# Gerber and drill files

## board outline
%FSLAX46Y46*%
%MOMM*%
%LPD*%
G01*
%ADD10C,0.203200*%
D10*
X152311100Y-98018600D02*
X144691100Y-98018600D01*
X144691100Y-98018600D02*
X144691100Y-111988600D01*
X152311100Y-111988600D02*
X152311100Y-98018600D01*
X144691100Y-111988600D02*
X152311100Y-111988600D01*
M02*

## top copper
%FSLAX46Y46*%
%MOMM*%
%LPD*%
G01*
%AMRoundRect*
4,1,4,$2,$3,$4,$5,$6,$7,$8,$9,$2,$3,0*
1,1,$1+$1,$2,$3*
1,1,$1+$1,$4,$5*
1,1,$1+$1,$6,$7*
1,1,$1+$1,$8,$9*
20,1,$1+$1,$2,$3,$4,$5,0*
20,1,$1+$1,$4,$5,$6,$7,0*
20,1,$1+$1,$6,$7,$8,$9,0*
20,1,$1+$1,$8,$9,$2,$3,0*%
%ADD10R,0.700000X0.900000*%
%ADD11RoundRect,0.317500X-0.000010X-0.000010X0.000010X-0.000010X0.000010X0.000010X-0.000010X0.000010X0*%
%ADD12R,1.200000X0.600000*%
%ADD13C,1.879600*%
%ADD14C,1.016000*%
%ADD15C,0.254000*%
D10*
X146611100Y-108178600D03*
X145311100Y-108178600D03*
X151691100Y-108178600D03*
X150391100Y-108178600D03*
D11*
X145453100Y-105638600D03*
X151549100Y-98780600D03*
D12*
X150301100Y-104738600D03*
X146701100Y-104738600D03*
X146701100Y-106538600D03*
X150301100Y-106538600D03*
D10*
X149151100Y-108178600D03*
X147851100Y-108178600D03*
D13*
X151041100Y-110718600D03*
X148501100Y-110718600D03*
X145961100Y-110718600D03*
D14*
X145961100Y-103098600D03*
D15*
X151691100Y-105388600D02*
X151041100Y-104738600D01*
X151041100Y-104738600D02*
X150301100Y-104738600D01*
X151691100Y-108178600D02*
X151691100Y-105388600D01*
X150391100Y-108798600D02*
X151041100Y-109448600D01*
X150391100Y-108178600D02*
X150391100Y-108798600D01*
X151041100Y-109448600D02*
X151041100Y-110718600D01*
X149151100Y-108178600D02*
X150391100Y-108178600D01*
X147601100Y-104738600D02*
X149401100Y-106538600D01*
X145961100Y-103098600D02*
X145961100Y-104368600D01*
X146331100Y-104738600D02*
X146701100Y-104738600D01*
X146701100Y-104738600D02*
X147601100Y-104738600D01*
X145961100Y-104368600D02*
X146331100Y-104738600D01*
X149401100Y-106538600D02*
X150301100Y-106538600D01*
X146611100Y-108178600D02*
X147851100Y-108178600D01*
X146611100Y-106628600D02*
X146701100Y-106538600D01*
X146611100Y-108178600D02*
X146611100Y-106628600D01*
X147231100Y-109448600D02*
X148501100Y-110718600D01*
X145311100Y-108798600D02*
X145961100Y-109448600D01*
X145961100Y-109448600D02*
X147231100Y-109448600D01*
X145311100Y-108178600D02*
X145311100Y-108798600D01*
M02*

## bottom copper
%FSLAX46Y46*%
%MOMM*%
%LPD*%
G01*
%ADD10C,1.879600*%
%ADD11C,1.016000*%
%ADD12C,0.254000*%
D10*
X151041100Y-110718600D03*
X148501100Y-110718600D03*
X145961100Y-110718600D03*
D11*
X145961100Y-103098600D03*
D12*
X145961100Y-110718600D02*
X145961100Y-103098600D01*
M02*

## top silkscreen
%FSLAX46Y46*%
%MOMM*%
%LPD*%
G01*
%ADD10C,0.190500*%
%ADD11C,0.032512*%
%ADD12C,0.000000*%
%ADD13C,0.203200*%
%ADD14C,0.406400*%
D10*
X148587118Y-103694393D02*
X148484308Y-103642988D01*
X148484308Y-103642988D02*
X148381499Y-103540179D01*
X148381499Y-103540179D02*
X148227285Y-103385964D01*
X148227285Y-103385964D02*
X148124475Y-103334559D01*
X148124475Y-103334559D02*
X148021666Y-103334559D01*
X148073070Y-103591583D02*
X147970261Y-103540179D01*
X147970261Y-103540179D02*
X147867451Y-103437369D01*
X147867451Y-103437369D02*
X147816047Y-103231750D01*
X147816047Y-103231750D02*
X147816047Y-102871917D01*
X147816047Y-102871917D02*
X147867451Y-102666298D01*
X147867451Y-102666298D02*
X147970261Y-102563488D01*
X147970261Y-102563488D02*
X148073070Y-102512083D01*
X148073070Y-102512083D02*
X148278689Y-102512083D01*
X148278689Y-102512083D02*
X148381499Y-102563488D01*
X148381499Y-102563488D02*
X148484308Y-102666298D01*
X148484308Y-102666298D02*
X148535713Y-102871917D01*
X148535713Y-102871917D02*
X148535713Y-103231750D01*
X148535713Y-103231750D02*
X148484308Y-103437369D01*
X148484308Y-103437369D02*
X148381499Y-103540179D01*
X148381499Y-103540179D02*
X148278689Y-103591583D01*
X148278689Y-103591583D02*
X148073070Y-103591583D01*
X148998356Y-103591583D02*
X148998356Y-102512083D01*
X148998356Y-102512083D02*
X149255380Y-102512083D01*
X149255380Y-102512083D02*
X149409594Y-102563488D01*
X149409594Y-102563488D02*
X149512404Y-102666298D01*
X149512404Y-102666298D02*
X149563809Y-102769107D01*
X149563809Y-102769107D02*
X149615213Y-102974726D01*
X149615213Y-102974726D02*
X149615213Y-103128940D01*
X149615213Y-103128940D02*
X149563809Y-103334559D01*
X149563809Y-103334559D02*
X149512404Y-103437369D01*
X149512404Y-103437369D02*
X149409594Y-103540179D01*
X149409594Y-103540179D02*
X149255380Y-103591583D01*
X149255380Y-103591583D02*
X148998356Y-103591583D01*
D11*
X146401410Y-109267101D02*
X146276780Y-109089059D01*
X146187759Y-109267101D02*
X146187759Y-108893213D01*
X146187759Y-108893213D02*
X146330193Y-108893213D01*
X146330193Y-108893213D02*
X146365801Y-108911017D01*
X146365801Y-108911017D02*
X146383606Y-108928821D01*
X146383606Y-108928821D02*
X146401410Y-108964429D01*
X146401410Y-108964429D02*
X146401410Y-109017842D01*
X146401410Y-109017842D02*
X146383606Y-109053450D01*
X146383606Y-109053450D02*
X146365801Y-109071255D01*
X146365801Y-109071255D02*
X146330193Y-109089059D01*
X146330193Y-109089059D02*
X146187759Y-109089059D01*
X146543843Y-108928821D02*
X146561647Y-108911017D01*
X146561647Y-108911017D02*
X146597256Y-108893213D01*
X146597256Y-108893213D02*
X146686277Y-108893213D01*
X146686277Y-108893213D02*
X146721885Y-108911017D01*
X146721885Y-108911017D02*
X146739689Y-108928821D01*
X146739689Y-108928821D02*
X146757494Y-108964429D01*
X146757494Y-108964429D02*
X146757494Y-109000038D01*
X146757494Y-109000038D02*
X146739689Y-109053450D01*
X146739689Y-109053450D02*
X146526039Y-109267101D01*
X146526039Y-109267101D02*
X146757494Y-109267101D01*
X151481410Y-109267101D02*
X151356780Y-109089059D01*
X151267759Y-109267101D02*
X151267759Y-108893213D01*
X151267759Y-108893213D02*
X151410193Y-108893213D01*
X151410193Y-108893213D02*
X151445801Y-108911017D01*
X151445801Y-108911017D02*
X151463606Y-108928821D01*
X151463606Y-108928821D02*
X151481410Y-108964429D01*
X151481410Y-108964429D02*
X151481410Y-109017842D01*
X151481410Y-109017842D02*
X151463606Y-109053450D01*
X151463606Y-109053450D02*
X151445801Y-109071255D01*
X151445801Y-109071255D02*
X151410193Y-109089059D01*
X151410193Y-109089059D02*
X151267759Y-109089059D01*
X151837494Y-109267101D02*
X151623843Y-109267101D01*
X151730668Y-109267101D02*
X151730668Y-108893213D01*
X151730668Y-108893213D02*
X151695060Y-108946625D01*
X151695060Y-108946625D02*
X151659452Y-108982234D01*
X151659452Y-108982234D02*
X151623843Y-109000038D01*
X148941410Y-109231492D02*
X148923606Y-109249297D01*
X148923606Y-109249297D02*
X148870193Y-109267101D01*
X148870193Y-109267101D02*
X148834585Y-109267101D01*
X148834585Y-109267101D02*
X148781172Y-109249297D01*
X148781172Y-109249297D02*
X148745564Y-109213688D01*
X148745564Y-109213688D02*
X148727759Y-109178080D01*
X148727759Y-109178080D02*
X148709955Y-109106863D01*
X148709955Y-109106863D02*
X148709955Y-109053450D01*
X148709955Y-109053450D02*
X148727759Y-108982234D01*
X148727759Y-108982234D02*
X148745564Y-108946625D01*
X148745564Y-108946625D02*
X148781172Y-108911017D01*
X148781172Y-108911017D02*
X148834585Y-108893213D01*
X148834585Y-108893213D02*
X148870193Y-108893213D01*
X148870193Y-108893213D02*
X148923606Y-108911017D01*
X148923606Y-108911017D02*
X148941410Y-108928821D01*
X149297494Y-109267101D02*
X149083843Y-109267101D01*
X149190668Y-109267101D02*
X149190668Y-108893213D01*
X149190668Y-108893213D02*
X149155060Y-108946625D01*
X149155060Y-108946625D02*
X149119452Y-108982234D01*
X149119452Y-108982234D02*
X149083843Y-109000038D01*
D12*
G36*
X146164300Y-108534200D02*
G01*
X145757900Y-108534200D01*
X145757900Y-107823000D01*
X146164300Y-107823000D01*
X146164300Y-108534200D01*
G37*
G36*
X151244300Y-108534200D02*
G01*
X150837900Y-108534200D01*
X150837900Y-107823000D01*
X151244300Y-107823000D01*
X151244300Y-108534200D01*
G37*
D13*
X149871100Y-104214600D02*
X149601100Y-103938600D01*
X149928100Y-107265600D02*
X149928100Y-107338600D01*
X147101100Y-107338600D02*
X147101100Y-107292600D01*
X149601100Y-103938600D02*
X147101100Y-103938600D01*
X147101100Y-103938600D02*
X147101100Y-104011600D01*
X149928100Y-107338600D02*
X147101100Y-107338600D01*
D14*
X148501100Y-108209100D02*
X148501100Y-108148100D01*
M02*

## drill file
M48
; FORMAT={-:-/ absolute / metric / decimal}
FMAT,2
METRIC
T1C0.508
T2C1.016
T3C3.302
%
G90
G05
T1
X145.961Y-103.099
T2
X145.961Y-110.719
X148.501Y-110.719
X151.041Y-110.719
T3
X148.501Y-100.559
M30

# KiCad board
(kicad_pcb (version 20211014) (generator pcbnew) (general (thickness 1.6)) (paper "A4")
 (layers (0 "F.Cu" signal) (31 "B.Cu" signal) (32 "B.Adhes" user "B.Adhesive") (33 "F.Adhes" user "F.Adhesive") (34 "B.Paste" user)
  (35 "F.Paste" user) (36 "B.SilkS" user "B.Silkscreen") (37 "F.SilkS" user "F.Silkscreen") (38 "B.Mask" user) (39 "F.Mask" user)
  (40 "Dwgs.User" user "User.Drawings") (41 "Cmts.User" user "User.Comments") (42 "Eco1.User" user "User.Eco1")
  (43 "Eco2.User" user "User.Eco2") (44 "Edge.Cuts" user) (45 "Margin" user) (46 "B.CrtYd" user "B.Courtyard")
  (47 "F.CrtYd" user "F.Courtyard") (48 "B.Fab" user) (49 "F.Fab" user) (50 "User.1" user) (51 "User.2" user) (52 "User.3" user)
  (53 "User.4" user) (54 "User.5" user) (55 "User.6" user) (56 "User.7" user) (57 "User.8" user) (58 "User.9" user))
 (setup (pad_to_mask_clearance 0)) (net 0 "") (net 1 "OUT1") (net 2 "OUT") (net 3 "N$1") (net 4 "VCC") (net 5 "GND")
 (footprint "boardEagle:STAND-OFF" (layer "F.Cu") (at 148.5011 100.5586)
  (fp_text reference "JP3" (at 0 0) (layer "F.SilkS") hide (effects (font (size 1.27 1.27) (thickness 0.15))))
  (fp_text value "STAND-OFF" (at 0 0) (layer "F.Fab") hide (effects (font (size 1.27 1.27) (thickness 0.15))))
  (pad "" np_thru_hole circle (at 0 0) (size 3.302 3.302) (drill 3.302) (layers *.Cu *.Mask)))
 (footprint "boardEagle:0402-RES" (layer "F.Cu") (at 145.9611 108.1786 180)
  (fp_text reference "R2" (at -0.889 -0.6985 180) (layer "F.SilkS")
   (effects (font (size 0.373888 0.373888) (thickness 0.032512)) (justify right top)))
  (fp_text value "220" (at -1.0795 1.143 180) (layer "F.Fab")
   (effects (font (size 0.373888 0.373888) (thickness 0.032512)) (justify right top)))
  (fp_poly (pts (xy -0.2032 0.3556) (xy 0.2032 0.3556) (xy 0.2032 -0.3556) (xy -0.2032 -0.3556)) (layer "F.SilkS") (width 0) (fill solid))
  (pad "1" smd rect (at -0.65 0 180) (size 0.7 0.9) (layers "F.Cu" "F.Paste" "F.Mask") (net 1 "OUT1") (solder_mask_margin 0.1016))
  (pad "2" smd rect (at 0.65 0 180) (size 0.7 0.9) (layers "F.Cu" "F.Paste" "F.Mask") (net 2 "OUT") (solder_mask_margin 0.1016)))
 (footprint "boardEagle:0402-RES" (layer "F.Cu") (at 151.0411 108.1786 180)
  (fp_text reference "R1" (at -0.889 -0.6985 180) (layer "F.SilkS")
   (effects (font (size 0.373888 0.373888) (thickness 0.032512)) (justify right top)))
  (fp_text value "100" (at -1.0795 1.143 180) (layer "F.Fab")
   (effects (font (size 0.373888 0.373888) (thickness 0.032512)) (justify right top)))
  (fp_poly (pts (xy -0.2032 0.3556) (xy 0.2032 0.3556) (xy 0.2032 -0.3556) (xy -0.2032 -0.3556)) (layer "F.SilkS") (width 0) (fill solid))
  (pad "1" smd rect (at -0.65 0 180) (size 0.7 0.9) (layers "F.Cu" "F.Paste" "F.Mask") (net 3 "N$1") (solder_mask_margin 0.1016))
  (pad "2" smd rect (at 0.65 0 180) (size 0.7 0.9) (layers "F.Cu" "F.Paste" "F.Mask") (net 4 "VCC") (solder_mask_margin 0.1016)))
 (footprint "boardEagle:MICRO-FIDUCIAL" (layer "F.Cu") (at 145.4531 105.6386)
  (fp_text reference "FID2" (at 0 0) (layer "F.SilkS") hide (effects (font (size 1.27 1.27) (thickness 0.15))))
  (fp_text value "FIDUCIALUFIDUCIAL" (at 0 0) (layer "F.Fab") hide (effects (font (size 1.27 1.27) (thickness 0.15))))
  (pad "1" smd roundrect (at 0 0) (size 0.635 0.635) (layers "F.Cu" "F.Mask") (roundrect_rratio 0.5) (solder_mask_margin 0.1016)))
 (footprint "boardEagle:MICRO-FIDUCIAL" (layer "F.Cu") (at 151.5491 98.7806)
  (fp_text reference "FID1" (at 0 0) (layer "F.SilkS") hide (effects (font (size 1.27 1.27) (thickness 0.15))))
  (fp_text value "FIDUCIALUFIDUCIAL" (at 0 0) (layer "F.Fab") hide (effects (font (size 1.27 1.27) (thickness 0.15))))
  (pad "1" smd roundrect (at 0 0) (size 0.635 0.635) (layers "F.Cu" "F.Mask") (roundrect_rratio 0.5) (solder_mask_margin 0.1016)))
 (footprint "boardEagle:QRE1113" (layer "F.Cu") (at 148.5011 105.6386 180)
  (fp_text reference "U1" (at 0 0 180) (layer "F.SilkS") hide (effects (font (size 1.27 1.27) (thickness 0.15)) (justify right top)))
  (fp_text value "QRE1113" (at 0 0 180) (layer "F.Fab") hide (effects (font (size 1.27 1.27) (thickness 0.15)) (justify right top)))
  (fp_line (start -1.37 1.424) (end -1.1 1.7) (layer "F.SilkS") (width 0.2032))
  (fp_line (start -1.427 -1.627) (end -1.427 -1.7) (layer "F.SilkS") (width 0.2032))
  (fp_line (start 1.4 -1.7) (end 1.4 -1.654) (layer "F.SilkS") (width 0.2032))
  (fp_line (start -1.1 1.7) (end 1.4 1.7) (layer "F.SilkS") (width 0.2032))
  (fp_line (start 1.4 1.7) (end 1.4 1.627) (layer "F.SilkS") (width 0.2032))
  (fp_line (start -1.427 -1.7) (end 1.4 -1.7) (layer "F.SilkS") (width 0.2032))
  (pad "1" smd rect (at -1.8 0.9 180) (size 1.2 0.6) (layers "F.Cu" "F.Paste" "F.Mask") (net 3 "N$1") (solder_mask_margin 0.1016))
  (pad "2" smd rect (at 1.8 0.9 180) (size 1.2 0.6) (layers "F.Cu" "F.Paste" "F.Mask") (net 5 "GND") (solder_mask_margin 0.1016))
  (pad "3" smd rect (at 1.8 -0.9 180) (size 1.2 0.6) (layers "F.Cu" "F.Paste" "F.Mask") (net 1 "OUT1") (solder_mask_margin 0.1016))
  (pad "4" smd rect (at -1.8 -0.9 180) (size 1.2 0.6) (layers "F.Cu" "F.Paste" "F.Mask") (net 5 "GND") (solder_mask_margin 0.1016)))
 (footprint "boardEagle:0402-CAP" (layer "F.Cu") (at 148.5011 108.1786 180)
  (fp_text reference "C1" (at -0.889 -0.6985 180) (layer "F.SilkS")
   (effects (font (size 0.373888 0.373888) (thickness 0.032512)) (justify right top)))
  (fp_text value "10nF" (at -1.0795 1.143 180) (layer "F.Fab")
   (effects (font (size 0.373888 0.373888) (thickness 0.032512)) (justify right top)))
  (fp_line (start 0 -0.0305) (end 0 0.0305) (layer "F.SilkS") (width 0.4064))
  (pad "1" smd rect (at -0.65 0 180) (size 0.7 0.9) (layers "F.Cu" "F.Paste" "F.Mask") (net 4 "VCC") (solder_mask_margin 0.1016))
  (pad "2" smd rect (at 0.65 0 180) (size 0.7 0.9) (layers "F.Cu" "F.Paste" "F.Mask") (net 1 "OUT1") (solder_mask_margin 0.1016)))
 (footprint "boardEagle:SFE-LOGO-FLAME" (layer "B.Cu") (at 149.3901 105.2576 180)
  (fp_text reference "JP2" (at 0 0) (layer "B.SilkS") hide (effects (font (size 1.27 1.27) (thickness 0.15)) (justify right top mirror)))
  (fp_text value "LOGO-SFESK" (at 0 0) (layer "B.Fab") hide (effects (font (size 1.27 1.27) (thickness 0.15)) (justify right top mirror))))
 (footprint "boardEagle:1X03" (layer "B.Cu") (at 151.0411 110.7186 180)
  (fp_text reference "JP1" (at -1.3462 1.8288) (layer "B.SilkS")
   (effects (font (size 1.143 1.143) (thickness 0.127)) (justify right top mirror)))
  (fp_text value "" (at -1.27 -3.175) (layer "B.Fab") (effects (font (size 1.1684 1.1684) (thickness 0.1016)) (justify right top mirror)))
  (pad "1" thru_hole circle (at 0 0 90) (size 1.8796 1.8796) (drill 1.016) (layers *.Cu *.Mask) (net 4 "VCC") (solder_mask_margin 0.1016))
  (pad "2" thru_hole circle (at 2.54 0 90) (size 1.8796 1.8796) (drill 1.016) (layers *.Cu *.Mask) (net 2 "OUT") (solder_mask_margin 0.1016))
  (pad "3" thru_hole circle (at 5.08 0 90) (size 1.8796 1.8796) (drill 1.016) (layers *.Cu *.Mask) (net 5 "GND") (solder_mask_margin 0.1016)))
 (gr_line (start 152.3111 98.0186) (end 144.6911 98.0186) (layer "Edge.Cuts") (width 0.2032))
 (gr_line (start 144.6911 98.0186) (end 144.6911 111.9886) (layer "Edge.Cuts") (width 0.2032))
 (gr_line (start 152.3111 111.9886) (end 152.3111 98.0186) (layer "Edge.Cuts") (width 0.2032))
 (gr_line (start 144.6911 111.9886) (end 152.3111 111.9886) (layer "Edge.Cuts") (width 0.2032))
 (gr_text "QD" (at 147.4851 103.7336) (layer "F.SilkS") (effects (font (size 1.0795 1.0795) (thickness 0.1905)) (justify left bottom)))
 (segment (start 151.6911 105.3886) (end 151.0411 104.7386) (width 0.254) (layer "F.Cu") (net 3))
 (segment (start 151.0411 104.7386) (end 150.3011 104.7386) (width 0.254) (layer "F.Cu") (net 3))
 (segment (start 151.6911 108.1786) (end 151.6911 105.3886) (width 0.254) (layer "F.Cu") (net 3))
 (segment (start 150.3911 108.7986) (end 151.0411 109.4486) (width 0.254) (layer "F.Cu") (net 4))
 (segment (start 150.3911 108.1786) (end 150.3911 108.7986) (width 0.254) (layer "F.Cu") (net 4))
 (segment (start 151.0411 109.4486) (end 151.0411 110.7186) (width 0.254) (layer "F.Cu") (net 4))
 (segment (start 149.1511 108.1786) (end 150.3911 108.1786) (width 0.254) (layer "F.Cu") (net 4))
 (segment (start 147.6011 104.7386) (end 149.4011 106.5386) (width 0.254) (layer "F.Cu") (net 5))
 (segment (start 145.9611 103.0986) (end 145.9611 104.3686) (width 0.254) (layer "F.Cu") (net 5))
 (segment (start 146.3311 104.7386) (end 146.7011 104.7386) (width 0.254) (layer "F.Cu") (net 5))
 (segment (start 146.7011 104.7386) (end 147.6011 104.7386) (width 0.254) (layer "F.Cu") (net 5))
 (segment (start 145.9611 104.3686) (end 146.3311 104.7386) (width 0.254) (layer "F.Cu") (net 5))
 (segment (start 149.4011 106.5386) (end 150.3011 106.5386) (width 0.254) (layer "F.Cu") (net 5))
 (via (at 145.9611 103.0986) (size 1.016) (drill 0.508) (layers "F.Cu" "B.Cu") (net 5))
 (segment (start 145.9611 110.7186) (end 145.9611 103.0986) (width 0.254) (layer "B.Cu") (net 5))
 (segment (start 146.6111 108.1786) (end 147.8511 108.1786) (width 0.254) (layer "F.Cu") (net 1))
 (segment (start 146.6111 106.6286) (end 146.7011 106.5386) (width 0.254) (layer "F.Cu") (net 1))
 (segment (start 146.6111 108.1786) (end 146.6111 106.6286) (width 0.254) (layer "F.Cu") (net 1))
 (segment (start 147.2311 109.4486) (end 148.5011 110.7186) (width 0.254) (layer "F.Cu") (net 2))
 (segment (start 145.3111 108.7986) (end 145.9611 109.4486) (width 0.254) (layer "F.Cu") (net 2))
 (segment (start 145.9611 109.4486) (end 147.2311 109.4486) (width 0.254) (layer "F.Cu") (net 2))
 (segment (start 145.3111 108.1786) (end 145.3111 108.7986) (width 0.254) (layer "F.Cu") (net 2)))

